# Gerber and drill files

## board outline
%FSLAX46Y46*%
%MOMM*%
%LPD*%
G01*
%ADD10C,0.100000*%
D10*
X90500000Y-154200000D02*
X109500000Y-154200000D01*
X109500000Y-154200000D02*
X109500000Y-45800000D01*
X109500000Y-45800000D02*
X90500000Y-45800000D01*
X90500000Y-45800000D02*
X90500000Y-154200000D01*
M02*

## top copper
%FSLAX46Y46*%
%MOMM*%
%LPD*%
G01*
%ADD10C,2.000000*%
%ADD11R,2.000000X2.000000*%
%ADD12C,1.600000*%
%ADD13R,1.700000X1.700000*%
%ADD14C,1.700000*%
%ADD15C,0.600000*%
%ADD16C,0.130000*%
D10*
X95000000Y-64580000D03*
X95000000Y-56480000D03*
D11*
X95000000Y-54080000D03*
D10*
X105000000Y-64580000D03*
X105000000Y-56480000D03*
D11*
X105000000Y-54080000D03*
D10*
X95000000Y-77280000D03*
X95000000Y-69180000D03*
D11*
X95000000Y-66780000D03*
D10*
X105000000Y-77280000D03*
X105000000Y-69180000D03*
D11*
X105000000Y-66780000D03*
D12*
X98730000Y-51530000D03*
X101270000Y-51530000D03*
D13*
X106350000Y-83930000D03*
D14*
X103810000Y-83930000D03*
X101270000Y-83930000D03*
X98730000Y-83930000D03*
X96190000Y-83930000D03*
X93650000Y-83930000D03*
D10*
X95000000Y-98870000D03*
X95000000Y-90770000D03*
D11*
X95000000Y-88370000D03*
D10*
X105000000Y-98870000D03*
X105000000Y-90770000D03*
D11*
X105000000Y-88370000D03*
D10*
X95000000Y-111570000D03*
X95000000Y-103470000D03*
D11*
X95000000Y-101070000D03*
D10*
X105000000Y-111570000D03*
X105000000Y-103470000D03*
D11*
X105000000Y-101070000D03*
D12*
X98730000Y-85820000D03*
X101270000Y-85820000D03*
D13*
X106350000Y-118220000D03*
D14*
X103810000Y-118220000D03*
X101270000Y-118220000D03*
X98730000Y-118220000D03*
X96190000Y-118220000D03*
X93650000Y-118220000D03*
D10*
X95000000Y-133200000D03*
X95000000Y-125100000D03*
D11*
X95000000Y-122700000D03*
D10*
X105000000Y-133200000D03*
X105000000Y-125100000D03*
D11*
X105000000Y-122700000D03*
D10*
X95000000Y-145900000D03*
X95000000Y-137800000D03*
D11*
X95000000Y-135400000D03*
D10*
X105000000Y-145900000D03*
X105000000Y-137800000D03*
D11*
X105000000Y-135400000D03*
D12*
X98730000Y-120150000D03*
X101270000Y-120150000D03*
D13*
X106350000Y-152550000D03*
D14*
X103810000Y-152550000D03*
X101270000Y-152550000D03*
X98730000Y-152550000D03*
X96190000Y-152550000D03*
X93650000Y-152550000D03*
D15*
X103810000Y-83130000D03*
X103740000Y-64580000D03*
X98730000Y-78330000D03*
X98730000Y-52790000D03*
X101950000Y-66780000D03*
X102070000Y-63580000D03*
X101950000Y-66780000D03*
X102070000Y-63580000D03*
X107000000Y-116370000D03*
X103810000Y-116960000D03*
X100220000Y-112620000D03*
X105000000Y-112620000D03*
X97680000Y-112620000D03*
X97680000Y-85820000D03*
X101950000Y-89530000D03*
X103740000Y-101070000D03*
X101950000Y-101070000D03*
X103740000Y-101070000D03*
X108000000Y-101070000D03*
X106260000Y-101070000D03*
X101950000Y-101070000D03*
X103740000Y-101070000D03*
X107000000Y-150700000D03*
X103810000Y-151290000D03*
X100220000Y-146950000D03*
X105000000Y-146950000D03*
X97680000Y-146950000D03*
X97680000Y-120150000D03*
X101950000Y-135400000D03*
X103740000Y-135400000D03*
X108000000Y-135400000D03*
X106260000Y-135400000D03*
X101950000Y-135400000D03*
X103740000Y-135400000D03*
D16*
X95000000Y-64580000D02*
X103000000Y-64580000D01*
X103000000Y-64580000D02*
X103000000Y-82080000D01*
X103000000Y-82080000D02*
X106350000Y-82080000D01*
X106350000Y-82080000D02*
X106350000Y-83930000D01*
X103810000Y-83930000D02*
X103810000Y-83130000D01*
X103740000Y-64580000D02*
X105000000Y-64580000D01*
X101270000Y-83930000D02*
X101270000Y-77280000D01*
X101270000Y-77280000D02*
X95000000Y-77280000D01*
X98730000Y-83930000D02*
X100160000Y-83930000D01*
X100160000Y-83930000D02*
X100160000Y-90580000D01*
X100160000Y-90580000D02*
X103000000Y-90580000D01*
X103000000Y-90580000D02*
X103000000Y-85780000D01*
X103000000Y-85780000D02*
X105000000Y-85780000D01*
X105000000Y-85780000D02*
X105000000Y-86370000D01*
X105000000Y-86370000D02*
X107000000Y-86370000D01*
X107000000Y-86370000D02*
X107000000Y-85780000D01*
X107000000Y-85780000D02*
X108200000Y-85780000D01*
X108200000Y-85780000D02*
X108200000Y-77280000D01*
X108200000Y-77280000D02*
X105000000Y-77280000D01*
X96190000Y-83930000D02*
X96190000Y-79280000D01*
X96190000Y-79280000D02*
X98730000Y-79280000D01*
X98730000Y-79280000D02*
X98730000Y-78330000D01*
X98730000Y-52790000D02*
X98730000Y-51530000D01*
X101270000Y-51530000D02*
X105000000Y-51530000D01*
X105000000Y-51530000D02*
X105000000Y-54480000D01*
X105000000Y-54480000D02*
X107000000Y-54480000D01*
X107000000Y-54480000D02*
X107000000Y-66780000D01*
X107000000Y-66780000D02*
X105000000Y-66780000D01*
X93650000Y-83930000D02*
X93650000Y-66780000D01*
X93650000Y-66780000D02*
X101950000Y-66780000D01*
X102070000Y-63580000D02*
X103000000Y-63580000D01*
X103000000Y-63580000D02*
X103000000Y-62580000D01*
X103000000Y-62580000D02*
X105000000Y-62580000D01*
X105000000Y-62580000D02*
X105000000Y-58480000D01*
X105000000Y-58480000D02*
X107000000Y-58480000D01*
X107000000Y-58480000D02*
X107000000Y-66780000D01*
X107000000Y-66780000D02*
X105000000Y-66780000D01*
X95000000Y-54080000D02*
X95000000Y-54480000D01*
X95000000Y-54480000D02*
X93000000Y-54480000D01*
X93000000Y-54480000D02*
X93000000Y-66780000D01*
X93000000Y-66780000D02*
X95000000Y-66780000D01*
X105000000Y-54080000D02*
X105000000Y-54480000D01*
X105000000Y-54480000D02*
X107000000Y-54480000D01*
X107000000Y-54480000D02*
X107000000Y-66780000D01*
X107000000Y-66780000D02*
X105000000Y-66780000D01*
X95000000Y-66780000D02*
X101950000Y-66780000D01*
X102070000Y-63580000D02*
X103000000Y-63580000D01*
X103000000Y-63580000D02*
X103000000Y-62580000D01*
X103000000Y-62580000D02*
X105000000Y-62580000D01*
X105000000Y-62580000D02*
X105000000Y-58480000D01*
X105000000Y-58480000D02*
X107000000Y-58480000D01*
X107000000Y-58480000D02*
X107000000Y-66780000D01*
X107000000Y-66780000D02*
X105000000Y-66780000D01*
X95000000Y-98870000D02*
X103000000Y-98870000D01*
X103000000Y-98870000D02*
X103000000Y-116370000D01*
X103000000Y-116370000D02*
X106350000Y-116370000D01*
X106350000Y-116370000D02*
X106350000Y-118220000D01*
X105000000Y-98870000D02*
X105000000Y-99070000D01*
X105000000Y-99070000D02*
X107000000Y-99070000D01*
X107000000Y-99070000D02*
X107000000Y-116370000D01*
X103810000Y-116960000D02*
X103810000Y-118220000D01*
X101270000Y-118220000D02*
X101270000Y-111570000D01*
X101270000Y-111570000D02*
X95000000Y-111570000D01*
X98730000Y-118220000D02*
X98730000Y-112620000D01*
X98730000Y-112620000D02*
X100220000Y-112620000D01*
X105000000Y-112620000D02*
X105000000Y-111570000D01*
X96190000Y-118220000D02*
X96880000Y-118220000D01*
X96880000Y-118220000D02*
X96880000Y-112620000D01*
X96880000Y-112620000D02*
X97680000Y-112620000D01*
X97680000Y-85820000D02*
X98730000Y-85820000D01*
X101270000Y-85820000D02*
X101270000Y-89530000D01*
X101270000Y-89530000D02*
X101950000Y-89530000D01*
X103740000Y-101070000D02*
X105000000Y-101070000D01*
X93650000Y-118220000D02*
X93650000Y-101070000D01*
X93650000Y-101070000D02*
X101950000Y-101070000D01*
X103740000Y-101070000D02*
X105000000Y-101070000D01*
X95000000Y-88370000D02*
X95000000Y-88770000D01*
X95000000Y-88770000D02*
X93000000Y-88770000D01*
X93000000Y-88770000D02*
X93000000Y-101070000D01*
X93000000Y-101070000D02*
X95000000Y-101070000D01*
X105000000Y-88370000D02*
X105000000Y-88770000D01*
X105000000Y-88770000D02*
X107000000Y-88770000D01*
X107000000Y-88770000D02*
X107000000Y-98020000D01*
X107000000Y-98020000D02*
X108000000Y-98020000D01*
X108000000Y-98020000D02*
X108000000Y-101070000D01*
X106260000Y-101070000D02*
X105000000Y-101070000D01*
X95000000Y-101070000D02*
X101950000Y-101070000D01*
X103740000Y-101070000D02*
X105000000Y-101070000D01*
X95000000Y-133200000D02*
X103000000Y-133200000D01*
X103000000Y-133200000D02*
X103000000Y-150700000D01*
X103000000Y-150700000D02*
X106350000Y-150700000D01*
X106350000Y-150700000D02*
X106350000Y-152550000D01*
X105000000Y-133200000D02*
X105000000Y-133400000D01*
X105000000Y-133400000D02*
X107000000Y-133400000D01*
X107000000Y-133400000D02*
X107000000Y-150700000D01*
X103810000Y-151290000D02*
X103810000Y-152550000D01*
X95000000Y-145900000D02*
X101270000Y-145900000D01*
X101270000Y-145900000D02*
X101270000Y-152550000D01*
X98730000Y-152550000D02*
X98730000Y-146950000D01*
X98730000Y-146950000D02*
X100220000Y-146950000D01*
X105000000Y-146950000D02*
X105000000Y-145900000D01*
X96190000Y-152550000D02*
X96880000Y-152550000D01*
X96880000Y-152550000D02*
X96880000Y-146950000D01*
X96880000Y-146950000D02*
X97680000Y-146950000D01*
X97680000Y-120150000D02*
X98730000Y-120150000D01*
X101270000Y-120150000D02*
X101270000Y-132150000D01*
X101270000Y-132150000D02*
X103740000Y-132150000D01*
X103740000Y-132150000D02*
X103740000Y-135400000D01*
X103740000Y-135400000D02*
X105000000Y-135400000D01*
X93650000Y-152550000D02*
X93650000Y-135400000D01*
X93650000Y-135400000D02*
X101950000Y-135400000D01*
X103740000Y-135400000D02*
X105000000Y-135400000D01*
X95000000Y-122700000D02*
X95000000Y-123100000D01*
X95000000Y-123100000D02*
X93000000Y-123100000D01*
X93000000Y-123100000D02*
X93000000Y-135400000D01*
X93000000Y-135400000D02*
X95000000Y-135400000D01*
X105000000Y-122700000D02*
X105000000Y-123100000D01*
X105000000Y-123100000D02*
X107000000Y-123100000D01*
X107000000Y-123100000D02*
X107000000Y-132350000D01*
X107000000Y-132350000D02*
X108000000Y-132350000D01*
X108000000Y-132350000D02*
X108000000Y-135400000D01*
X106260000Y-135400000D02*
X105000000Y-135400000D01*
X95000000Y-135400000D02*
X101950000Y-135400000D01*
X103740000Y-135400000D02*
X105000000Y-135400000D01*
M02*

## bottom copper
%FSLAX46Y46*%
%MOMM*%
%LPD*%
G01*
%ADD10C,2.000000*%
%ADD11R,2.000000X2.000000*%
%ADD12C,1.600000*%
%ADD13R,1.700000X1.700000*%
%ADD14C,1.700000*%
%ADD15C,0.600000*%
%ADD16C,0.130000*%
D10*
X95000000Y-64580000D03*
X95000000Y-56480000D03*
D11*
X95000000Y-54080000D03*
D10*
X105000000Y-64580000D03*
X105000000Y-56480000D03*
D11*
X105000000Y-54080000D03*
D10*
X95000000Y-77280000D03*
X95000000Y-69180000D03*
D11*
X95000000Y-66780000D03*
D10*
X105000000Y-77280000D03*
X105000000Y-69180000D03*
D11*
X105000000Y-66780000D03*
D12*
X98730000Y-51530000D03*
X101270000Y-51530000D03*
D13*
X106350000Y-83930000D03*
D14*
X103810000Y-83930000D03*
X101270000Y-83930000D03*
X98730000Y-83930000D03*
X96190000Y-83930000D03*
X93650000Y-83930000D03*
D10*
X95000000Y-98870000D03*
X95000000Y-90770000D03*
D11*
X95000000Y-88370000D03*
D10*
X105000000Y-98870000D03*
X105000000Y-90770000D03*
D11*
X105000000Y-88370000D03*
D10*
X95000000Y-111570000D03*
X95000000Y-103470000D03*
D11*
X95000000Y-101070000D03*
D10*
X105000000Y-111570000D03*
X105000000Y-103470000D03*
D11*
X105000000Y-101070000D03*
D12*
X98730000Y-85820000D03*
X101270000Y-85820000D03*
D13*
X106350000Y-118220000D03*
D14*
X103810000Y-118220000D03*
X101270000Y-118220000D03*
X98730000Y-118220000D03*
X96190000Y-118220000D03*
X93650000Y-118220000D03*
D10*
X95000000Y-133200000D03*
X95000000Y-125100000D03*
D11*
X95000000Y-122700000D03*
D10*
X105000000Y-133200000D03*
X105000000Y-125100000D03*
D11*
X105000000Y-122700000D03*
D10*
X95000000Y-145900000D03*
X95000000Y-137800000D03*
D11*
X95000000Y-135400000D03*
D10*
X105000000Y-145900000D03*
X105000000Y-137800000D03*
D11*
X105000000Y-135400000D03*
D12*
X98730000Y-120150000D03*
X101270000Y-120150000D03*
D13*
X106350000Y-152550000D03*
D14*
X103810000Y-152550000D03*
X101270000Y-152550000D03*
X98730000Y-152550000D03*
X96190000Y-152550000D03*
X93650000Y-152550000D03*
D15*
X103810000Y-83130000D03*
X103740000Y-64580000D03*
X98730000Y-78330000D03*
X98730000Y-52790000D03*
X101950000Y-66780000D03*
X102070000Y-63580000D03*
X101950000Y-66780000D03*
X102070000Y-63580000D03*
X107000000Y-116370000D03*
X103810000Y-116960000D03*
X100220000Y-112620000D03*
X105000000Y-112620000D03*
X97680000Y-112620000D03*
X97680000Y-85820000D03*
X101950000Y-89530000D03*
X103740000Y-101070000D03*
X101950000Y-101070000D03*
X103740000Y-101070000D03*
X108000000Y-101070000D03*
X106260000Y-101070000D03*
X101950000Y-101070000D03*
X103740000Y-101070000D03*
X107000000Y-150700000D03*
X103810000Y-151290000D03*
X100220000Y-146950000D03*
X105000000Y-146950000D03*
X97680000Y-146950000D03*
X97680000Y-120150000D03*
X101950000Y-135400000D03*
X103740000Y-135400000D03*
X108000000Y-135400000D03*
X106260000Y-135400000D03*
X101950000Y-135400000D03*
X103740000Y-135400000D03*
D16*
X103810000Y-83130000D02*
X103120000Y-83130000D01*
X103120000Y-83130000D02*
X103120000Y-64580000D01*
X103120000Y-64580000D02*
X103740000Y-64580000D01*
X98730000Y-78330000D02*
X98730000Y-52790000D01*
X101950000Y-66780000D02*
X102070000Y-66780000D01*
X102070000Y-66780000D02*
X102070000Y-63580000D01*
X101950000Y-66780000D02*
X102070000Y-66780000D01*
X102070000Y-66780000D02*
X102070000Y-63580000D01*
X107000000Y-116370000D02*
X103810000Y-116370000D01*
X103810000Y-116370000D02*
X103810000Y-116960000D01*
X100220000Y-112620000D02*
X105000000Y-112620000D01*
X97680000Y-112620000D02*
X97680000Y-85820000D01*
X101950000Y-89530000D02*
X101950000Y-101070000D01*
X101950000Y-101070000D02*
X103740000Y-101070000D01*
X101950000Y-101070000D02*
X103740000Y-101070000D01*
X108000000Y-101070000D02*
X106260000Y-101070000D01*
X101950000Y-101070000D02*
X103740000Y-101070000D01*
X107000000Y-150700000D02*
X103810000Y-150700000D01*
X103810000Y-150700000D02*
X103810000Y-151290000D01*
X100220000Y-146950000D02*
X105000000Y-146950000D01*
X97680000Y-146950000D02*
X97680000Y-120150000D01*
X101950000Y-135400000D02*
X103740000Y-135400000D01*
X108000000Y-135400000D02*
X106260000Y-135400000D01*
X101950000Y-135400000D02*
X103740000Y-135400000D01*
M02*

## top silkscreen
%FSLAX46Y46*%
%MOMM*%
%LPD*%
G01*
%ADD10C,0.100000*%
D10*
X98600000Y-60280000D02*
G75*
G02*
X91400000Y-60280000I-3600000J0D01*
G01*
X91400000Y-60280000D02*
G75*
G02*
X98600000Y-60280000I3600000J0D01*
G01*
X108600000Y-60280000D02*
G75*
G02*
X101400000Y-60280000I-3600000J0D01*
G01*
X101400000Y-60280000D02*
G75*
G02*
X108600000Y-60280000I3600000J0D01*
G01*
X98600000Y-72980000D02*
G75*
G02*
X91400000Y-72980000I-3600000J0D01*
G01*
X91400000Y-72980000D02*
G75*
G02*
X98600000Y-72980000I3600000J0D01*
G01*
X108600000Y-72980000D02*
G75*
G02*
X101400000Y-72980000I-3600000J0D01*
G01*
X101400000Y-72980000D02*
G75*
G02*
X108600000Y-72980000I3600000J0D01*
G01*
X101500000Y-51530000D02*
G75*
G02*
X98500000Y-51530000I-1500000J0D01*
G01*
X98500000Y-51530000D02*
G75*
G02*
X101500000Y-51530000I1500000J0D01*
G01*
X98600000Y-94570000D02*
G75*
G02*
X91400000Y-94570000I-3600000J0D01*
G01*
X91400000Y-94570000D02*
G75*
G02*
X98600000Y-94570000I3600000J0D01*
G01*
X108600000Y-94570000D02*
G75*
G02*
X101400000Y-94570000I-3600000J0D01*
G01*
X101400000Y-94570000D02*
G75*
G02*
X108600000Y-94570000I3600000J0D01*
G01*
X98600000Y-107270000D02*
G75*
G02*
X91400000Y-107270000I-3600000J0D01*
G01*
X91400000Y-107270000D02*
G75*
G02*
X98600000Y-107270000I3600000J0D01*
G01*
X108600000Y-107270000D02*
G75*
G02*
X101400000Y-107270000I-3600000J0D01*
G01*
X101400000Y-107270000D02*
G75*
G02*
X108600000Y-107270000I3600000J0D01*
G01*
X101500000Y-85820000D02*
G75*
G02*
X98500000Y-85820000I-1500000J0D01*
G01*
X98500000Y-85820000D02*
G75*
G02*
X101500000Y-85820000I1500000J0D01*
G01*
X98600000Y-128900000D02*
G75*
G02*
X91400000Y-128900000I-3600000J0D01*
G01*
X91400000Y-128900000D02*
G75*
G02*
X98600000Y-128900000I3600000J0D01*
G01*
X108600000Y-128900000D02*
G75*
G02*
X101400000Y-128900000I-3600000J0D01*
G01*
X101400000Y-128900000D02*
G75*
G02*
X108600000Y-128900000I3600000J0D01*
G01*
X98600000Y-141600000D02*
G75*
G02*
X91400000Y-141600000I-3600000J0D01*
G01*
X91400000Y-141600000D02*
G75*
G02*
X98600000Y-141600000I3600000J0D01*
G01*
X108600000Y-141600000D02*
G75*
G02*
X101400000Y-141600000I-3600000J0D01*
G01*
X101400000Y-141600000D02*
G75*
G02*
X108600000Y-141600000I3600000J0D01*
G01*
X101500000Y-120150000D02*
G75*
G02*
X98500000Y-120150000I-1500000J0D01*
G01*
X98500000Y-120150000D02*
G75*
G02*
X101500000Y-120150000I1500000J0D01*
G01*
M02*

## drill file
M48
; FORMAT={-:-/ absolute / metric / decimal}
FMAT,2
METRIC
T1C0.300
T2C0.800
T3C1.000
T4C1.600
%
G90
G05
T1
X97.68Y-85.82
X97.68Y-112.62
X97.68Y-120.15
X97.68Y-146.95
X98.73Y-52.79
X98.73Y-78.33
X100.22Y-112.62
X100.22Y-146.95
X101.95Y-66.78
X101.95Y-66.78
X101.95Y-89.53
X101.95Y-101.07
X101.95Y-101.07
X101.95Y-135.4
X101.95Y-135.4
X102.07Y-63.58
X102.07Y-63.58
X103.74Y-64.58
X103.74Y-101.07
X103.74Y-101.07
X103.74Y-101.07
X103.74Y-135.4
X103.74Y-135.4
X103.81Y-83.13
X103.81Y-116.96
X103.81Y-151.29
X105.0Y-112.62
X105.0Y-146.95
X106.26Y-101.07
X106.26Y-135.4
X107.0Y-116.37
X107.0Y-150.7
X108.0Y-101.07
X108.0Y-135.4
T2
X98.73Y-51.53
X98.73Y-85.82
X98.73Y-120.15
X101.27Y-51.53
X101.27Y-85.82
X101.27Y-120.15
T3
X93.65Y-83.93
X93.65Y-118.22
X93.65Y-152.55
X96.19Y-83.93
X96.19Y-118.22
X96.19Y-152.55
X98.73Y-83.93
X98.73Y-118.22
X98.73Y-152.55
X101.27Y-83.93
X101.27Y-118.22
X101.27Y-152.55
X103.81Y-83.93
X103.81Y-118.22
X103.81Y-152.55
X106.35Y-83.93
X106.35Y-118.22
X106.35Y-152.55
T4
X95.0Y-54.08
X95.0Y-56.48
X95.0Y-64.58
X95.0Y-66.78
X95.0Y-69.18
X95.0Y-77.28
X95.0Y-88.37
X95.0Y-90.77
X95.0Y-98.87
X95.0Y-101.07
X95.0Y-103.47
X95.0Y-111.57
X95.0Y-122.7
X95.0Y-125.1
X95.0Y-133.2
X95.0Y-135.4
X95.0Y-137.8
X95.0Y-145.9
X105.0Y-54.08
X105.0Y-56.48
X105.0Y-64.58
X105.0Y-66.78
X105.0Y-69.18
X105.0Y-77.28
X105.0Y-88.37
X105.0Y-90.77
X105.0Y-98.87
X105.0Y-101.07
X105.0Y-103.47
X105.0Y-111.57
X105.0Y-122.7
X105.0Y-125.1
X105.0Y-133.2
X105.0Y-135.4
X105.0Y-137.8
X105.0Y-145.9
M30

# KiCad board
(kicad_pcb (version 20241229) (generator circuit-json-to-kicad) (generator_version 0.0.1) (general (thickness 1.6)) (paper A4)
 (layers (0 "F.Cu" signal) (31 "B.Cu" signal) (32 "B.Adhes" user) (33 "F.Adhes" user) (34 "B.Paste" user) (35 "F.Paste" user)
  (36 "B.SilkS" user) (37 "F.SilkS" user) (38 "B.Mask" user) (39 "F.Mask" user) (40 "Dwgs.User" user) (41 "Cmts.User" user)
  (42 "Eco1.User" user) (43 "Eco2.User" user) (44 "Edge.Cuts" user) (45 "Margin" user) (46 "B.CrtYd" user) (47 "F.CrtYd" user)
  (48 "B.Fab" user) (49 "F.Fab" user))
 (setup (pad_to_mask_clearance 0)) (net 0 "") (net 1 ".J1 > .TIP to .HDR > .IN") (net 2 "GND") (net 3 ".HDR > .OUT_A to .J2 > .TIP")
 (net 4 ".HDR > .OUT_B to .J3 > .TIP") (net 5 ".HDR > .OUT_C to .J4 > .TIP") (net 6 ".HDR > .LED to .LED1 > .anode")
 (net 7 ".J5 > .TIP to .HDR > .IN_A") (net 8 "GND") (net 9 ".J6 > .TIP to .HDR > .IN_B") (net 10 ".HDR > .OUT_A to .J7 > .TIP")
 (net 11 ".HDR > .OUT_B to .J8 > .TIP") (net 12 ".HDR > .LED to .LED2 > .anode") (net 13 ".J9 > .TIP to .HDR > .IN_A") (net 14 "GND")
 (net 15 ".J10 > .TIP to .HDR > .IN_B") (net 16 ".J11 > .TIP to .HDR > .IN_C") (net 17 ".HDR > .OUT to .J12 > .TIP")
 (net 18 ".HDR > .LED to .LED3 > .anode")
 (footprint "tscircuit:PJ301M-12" (layer F.Cu) (at 95 59.33 0)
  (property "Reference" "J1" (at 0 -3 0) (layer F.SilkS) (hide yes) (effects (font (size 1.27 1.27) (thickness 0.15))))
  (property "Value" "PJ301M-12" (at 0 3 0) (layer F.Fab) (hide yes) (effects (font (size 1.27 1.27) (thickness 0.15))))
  (fp_circle (center 0 0.9500000000000028) (end 3.6 0.9500000000000028) (layer F.SilkS) (stroke (width 0.1) (type default)) (fill no))
  (pad "1" thru_hole circle (at 0 5.25 0) (size 2 2) (drill 1.6) (layers *.Cu *.Mask) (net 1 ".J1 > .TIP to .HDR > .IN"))
  (pad "2" thru_hole circle (at 0 -2.8499999999999943 0) (size 2 2) (drill 1.6) (layers *.Cu *.Mask))
  (pad "3" thru_hole rect (at 0 -5.25 0) (size 2 2) (drill 1.6) (layers *.Cu *.Mask) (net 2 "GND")))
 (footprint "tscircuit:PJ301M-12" (layer F.Cu) (at 105 59.33 0)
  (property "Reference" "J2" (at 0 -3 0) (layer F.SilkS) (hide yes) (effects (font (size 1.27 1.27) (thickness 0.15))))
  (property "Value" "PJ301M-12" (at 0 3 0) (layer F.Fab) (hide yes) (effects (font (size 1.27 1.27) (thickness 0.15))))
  (fp_circle (center 0 0.9500000000000028) (end 3.6 0.9500000000000028) (layer F.SilkS) (stroke (width 0.1) (type default)) (fill no))
  (pad "1" thru_hole circle (at 0 5.25 0) (size 2 2) (drill 1.6) (layers *.Cu *.Mask) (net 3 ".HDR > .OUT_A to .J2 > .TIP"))
  (pad "2" thru_hole circle (at 0 -2.8499999999999943 0) (size 2 2) (drill 1.6) (layers *.Cu *.Mask))
  (pad "3" thru_hole rect (at 0 -5.25 0) (size 2 2) (drill 1.6) (layers *.Cu *.Mask) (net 2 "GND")))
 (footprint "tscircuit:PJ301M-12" (layer F.Cu) (at 95 72.03 0)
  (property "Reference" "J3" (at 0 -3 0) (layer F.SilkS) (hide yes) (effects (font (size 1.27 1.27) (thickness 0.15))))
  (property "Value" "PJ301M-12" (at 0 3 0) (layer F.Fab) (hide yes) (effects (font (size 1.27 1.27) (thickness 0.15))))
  (fp_circle (center 0 0.9500000000000028) (end 3.6 0.9500000000000028) (layer F.SilkS) (stroke (width 0.1) (type default)) (fill no))
  (pad "1" thru_hole circle (at 0 5.2500000000000036 0) (size 2 2) (drill 1.6) (layers *.Cu *.Mask) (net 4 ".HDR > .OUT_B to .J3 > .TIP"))
  (pad "2" thru_hole circle (at 0 -2.849999999999998 0) (size 2 2) (drill 1.6) (layers *.Cu *.Mask))
  (pad "3" thru_hole rect (at 0 -5.25 0) (size 2 2) (drill 1.6) (layers *.Cu *.Mask) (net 2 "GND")))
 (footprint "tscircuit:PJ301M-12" (layer F.Cu) (at 105 72.03 0)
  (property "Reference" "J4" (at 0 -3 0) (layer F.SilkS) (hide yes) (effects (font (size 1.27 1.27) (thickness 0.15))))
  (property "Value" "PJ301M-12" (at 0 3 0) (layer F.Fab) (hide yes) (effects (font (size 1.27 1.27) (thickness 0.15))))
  (fp_circle (center 0 0.9500000000000028) (end 3.6 0.9500000000000028) (layer F.SilkS) (stroke (width 0.1) (type default)) (fill no))
  (pad "1" thru_hole circle (at 0 5.2500000000000036 0) (size 2 2) (drill 1.6) (layers *.Cu *.Mask) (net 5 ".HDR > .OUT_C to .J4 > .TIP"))
  (pad "2" thru_hole circle (at 0 -2.849999999999998 0) (size 2 2) (drill 1.6) (layers *.Cu *.Mask))
  (pad "3" thru_hole rect (at 0 -5.25 0) (size 2 2) (drill 1.6) (layers *.Cu *.Mask) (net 2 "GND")))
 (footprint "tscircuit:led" (layer F.Cu) (at 100 51.53 0)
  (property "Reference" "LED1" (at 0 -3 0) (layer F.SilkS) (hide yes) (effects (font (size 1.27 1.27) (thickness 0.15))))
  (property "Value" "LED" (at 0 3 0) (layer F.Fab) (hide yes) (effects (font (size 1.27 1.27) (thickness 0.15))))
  (fp_circle (center 0 0) (end 1.5 0) (layer F.SilkS) (stroke (width 0.1) (type default)) (fill no))
  (pad "1" thru_hole circle (at -1.27 0 0) (size 1.6 1.6) (drill 0.8) (layers *.Cu *.Mask) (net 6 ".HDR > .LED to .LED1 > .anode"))
  (pad "2" thru_hole circle (at 1.27 0 0) (size 1.6 1.6) (drill 0.8) (layers *.Cu *.Mask) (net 2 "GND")))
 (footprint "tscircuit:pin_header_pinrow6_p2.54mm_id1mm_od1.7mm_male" (layer F.Cu) (at 100 83.93 0)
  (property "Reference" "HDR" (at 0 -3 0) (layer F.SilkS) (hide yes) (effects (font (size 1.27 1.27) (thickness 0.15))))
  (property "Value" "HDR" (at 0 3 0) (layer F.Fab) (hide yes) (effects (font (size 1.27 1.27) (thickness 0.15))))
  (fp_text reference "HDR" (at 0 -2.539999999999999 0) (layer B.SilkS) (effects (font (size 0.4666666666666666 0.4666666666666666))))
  (pad "1" thru_hole rect (at 6.35 0 180) (size 1.7 1.7) (drill 1) (layers *.Cu *.Mask) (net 1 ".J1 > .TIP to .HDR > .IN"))
  (pad "2" thru_hole circle (at 3.8099999999999996 0 0) (size 1.7 1.7) (drill 1) (layers *.Cu *.Mask) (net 3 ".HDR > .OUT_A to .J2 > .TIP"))
  (pad "3" thru_hole circle (at 1.2699999999999996 0 0) (size 1.7 1.7) (drill 1) (layers *.Cu *.Mask) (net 4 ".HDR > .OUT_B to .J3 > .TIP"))
  (pad "4" thru_hole circle (at -1.2700000000000005 0 0) (size 1.7 1.7) (drill 1) (layers *.Cu *.Mask) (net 5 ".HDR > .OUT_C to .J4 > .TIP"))
  (pad "5" thru_hole circle (at -3.8100000000000005 0 0) (size 1.7 1.7) (drill 1) (layers *.Cu *.Mask)
   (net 6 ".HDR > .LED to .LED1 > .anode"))
  (pad "6" thru_hole circle (at -6.35 0 0) (size 1.7 1.7) (drill 1) (layers *.Cu *.Mask) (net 2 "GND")))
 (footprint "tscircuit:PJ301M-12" (layer F.Cu) (at 95 93.62 0)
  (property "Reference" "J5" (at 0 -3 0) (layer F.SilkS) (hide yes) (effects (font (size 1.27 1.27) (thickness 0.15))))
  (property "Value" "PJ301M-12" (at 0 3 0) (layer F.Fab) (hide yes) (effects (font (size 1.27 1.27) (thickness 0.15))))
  (fp_circle (center 0 0.9499999999999993) (end 3.6 0.9499999999999993) (layer F.SilkS) (stroke (width 0.1) (type default)) (fill no))
  (pad "1" thru_hole circle (at 0 5.249999999999999 0) (size 2 2) (drill 1.6) (layers *.Cu *.Mask) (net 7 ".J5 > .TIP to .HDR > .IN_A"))
  (pad "2" thru_hole circle (at 0 -2.8500000000000014 0) (size 2 2) (drill 1.6) (layers *.Cu *.Mask))
  (pad "3" thru_hole rect (at 0 -5.25 0) (size 2 2) (drill 1.6) (layers *.Cu *.Mask) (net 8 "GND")))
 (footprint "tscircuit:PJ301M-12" (layer F.Cu) (at 105 93.62 0)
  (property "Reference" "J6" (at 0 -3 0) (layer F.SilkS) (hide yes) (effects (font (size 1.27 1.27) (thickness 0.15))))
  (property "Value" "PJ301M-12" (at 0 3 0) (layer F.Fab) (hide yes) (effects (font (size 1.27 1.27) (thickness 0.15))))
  (fp_circle (center 0 0.9499999999999993) (end 3.6 0.9499999999999993) (layer F.SilkS) (stroke (width 0.1) (type default)) (fill no))
  (pad "1" thru_hole circle (at 0 5.249999999999999 0) (size 2 2) (drill 1.6) (layers *.Cu *.Mask) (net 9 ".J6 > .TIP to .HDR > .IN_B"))
  (pad "2" thru_hole circle (at 0 -2.8500000000000014 0) (size 2 2) (drill 1.6) (layers *.Cu *.Mask))
  (pad "3" thru_hole rect (at 0 -5.25 0) (size 2 2) (drill 1.6) (layers *.Cu *.Mask) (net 8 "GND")))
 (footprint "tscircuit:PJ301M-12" (layer F.Cu) (at 95 106.32 0)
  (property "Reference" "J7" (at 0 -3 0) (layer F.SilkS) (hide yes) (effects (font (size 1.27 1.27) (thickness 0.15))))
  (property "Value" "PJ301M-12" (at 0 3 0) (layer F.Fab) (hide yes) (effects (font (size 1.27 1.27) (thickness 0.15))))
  (fp_circle (center 0 0.9499999999999993) (end 3.6 0.9499999999999993) (layer F.SilkS) (stroke (width 0.1) (type default)) (fill no))
  (pad "1" thru_hole circle (at 0 5.25 0) (size 2 2) (drill 1.6) (layers *.Cu *.Mask) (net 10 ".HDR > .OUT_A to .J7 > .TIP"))
  (pad "2" thru_hole circle (at 0 -2.8500000000000005 0) (size 2 2) (drill 1.6) (layers *.Cu *.Mask))
  (pad "3" thru_hole rect (at 0 -5.250000000000001 0) (size 2 2) (drill 1.6) (layers *.Cu *.Mask) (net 8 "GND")))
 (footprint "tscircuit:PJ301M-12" (layer F.Cu) (at 105 106.32 0)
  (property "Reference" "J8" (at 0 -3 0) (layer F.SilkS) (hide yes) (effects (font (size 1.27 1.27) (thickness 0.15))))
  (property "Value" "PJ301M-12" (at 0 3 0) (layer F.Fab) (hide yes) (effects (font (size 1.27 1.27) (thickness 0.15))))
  (fp_circle (center 0 0.9499999999999993) (end 3.6 0.9499999999999993) (layer F.SilkS) (stroke (width 0.1) (type default)) (fill no))
  (pad "1" thru_hole circle (at 0 5.25 0) (size 2 2) (drill 1.6) (layers *.Cu *.Mask) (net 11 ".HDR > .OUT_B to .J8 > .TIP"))
  (pad "2" thru_hole circle (at 0 -2.8500000000000005 0) (size 2 2) (drill 1.6) (layers *.Cu *.Mask))
  (pad "3" thru_hole rect (at 0 -5.250000000000001 0) (size 2 2) (drill 1.6) (layers *.Cu *.Mask) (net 8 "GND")))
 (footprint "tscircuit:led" (layer F.Cu) (at 100 85.82 0)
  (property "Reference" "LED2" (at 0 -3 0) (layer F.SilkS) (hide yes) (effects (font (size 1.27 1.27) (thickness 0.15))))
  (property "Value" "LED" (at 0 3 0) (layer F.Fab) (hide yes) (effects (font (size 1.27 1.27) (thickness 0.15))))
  (fp_circle (center 0 0) (end 1.5 0) (layer F.SilkS) (stroke (width 0.1) (type default)) (fill no))
  (pad "1" thru_hole circle (at -1.27 0 0) (size 1.6 1.6) (drill 0.8) (layers *.Cu *.Mask) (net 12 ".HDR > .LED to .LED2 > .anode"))
  (pad "2" thru_hole circle (at 1.27 0 0) (size 1.6 1.6) (drill 0.8) (layers *.Cu *.Mask) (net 8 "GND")))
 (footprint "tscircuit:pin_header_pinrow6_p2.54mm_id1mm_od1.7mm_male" (layer F.Cu) (at 100 118.22 0)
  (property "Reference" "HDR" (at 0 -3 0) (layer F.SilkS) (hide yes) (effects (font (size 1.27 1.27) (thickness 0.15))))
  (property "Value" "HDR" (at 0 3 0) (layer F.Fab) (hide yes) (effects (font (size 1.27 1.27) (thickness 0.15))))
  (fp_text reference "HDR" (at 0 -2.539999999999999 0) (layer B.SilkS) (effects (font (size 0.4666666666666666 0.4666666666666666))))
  (pad "1" thru_hole rect (at 6.35 0 180) (size 1.7 1.7) (drill 1) (layers *.Cu *.Mask) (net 7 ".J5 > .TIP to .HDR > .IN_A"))
  (pad "2" thru_hole circle (at 3.8099999999999996 0 0) (size 1.7 1.7) (drill 1) (layers *.Cu *.Mask) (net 9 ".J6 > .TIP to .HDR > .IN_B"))
  (pad "3" thru_hole circle (at 1.2699999999999996 0 0) (size 1.7 1.7) (drill 1) (layers *.Cu *.Mask) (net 10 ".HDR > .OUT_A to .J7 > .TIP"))
  (pad "4" thru_hole circle (at -1.2700000000000005 0 0) (size 1.7 1.7) (drill 1) (layers *.Cu *.Mask)
   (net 11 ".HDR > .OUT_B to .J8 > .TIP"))
  (pad "5" thru_hole circle (at -3.8100000000000005 0 0) (size 1.7 1.7) (drill 1) (layers *.Cu *.Mask)
   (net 12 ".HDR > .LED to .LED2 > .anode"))
  (pad "6" thru_hole circle (at -6.35 0 0) (size 1.7 1.7) (drill 1) (layers *.Cu *.Mask) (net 8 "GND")))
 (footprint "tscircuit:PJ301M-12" (layer F.Cu) (at 95 127.94999999999999 0)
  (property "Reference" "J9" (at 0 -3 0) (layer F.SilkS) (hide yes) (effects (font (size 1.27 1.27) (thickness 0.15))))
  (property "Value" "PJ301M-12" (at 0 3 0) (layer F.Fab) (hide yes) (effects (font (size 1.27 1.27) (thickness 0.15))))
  (fp_circle (center 0 0.9500000000000028) (end 3.6 0.9500000000000028) (layer F.SilkS) (stroke (width 0.1) (type default)) (fill no))
  (pad "1" thru_hole circle (at 0 5.25 0) (size 2 2) (drill 1.6) (layers *.Cu *.Mask) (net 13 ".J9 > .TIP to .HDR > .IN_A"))
  (pad "2" thru_hole circle (at 0 -2.849999999999998 0) (size 2 2) (drill 1.6) (layers *.Cu *.Mask))
  (pad "3" thru_hole rect (at 0 -5.2499999999999964 0) (size 2 2) (drill 1.6) (layers *.Cu *.Mask) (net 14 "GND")))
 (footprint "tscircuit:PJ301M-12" (layer F.Cu) (at 105 127.94999999999999 0)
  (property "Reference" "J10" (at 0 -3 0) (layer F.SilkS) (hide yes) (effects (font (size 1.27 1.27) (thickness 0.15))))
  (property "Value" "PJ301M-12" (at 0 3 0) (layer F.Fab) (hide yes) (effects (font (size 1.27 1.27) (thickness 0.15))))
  (fp_circle (center 0 0.9500000000000028) (end 3.6 0.9500000000000028) (layer F.SilkS) (stroke (width 0.1) (type default)) (fill no))
  (pad "1" thru_hole circle (at 0 5.25 0) (size 2 2) (drill 1.6) (layers *.Cu *.Mask) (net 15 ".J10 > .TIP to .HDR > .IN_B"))
  (pad "2" thru_hole circle (at 0 -2.849999999999998 0) (size 2 2) (drill 1.6) (layers *.Cu *.Mask))
  (pad "3" thru_hole rect (at 0 -5.2499999999999964 0) (size 2 2) (drill 1.6) (layers *.Cu *.Mask) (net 14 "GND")))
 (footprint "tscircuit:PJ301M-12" (layer F.Cu) (at 95 140.65 0)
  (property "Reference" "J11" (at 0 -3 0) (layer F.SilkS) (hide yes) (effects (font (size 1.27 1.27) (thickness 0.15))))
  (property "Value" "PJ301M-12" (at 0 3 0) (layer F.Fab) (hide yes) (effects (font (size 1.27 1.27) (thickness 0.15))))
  (fp_circle (center 0 0.9500000000000028) (end 3.6 0.9500000000000028) (layer F.SilkS) (stroke (width 0.1) (type default)) (fill no))
  (pad "1" thru_hole circle (at 0 5.25 0) (size 2 2) (drill 1.6) (layers *.Cu *.Mask) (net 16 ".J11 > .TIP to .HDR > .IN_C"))
  (pad "2" thru_hole circle (at 0 -2.8499999999999943 0) (size 2 2) (drill 1.6) (layers *.Cu *.Mask))
  (pad "3" thru_hole rect (at 0 -5.25 0) (size 2 2) (drill 1.6) (layers *.Cu *.Mask) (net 14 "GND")))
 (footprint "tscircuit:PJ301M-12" (layer F.Cu) (at 105 140.65 0)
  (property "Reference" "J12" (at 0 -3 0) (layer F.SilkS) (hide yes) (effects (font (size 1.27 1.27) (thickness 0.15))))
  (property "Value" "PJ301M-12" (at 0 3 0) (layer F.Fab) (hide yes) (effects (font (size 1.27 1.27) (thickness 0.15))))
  (fp_circle (center 0 0.9500000000000028) (end 3.6 0.9500000000000028) (layer F.SilkS) (stroke (width 0.1) (type default)) (fill no))
  (pad "1" thru_hole circle (at 0 5.25 0) (size 2 2) (drill 1.6) (layers *.Cu *.Mask) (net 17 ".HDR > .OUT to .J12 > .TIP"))
  (pad "2" thru_hole circle (at 0 -2.8499999999999943 0) (size 2 2) (drill 1.6) (layers *.Cu *.Mask))
  (pad "3" thru_hole rect (at 0 -5.25 0) (size 2 2) (drill 1.6) (layers *.Cu *.Mask) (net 14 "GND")))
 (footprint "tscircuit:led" (layer F.Cu) (at 100 120.15 0)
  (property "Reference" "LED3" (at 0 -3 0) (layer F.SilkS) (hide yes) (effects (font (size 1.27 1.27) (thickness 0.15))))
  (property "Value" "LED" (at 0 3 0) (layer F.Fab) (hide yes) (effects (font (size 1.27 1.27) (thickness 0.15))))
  (fp_circle (center 0 0) (end 1.5 0) (layer F.SilkS) (stroke (width 0.1) (type default)) (fill no))
  (pad "1" thru_hole circle (at -1.27 0 0) (size 1.6 1.6) (drill 0.8) (layers *.Cu *.Mask) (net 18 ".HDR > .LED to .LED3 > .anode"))
  (pad "2" thru_hole circle (at 1.27 0 0) (size 1.6 1.6) (drill 0.8) (layers *.Cu *.Mask) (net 14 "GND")))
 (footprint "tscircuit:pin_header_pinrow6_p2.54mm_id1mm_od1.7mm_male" (layer F.Cu) (at 100 152.55 0)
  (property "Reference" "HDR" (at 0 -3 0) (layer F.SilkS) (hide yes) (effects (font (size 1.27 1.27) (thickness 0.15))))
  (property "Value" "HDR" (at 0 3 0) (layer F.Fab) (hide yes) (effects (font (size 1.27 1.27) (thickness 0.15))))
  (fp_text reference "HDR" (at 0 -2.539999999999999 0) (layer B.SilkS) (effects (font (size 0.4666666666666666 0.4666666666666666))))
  (pad "1" thru_hole rect (at 6.35 0 180) (size 1.7 1.7) (drill 1) (layers *.Cu *.Mask) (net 13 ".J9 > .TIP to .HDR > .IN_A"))
  (pad "2" thru_hole circle (at 3.8099999999999996 0 0) (size 1.7 1.7) (drill 1) (layers *.Cu *.Mask) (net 15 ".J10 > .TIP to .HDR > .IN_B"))
  (pad "3" thru_hole circle (at 1.2699999999999996 0 0) (size 1.7 1.7) (drill 1) (layers *.Cu *.Mask) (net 16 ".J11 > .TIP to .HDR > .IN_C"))
  (pad "4" thru_hole circle (at -1.2700000000000005 0 0) (size 1.7 1.7) (drill 1) (layers *.Cu *.Mask) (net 17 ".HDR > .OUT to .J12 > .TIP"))
  (pad "5" thru_hole circle (at -3.8100000000000005 0 0) (size 1.7 1.7) (drill 1) (layers *.Cu *.Mask)
   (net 18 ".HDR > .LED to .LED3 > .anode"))
  (pad "6" thru_hole circle (at -6.35 0 0) (size 1.7 1.7) (drill 1) (layers *.Cu *.Mask) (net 14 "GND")))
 (segment (start 95 64.58) (end 103 64.58) (width 0.13) (layer F.Cu) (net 1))
 (segment (start 103 64.58) (end 103 82.08) (width 0.13) (layer F.Cu) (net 1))
 (segment (start 103 82.08) (end 106.35 82.08) (width 0.13) (layer F.Cu) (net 1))
 (segment (start 106.35 82.08) (end 106.35 83.93) (width 0.13) (layer F.Cu) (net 1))
 (segment (start 103.81 83.93) (end 103.81 83.13) (width 0.13) (layer F.Cu) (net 3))
 (segment (start 103.81 83.13) (end 103.12 83.13) (width 0.13) (layer B.Cu) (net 3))
 (segment (start 103.12 83.13) (end 103.12 64.58) (width 0.13) (layer B.Cu) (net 3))
 (segment (start 103.12 64.58) (end 103.74 64.58) (width 0.13) (layer B.Cu) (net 3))
 (segment (start 103.74 64.58) (end 105 64.58) (width 0.13) (layer F.Cu) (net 3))
 (segment (start 101.27 83.93) (end 101.27 77.28) (width 0.13) (layer F.Cu) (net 4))
 (segment (start 101.27 77.28) (end 95 77.28) (width 0.13) (layer F.Cu) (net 4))
 (segment (start 98.73 83.93) (end 100.16 83.93) (width 0.13) (layer F.Cu) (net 5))
 (segment (start 100.16 83.93) (end 100.16 90.58) (width 0.13) (layer F.Cu) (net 5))
 (segment (start 100.16 90.58) (end 103 90.58) (width 0.13) (layer F.Cu) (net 5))
 (segment (start 103 90.58) (end 103 85.78) (width 0.13) (layer F.Cu) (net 5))
 (segment (start 103 85.78) (end 105 85.78) (width 0.13) (layer F.Cu) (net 5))
 (segment (start 105 85.78) (end 105 86.37) (width 0.13) (layer F.Cu) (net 5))
 (segment (start 105 86.37) (end 107 86.37) (width 0.13) (layer F.Cu) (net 5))
 (segment (start 107 86.37) (end 107 85.78) (width 0.13) (layer F.Cu) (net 5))
 (segment (start 107 85.78) (end 108.2 85.78) (width 0.13) (layer F.Cu) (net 5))
 (segment (start 108.2 85.78) (end 108.2 77.28) (width 0.13) (layer F.Cu) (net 5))
 (segment (start 108.2 77.28) (end 105 77.28) (width 0.13) (layer F.Cu) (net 5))
 (segment (start 96.19 83.93) (end 96.19 79.28) (width 0.13) (layer F.Cu) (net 6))
 (segment (start 96.19 79.28) (end 98.73 79.28) (width 0.13) (layer F.Cu) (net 6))
 (segment (start 98.73 79.28) (end 98.73 78.33000000000001) (width 0.13) (layer F.Cu) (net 6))
 (segment (start 98.73 78.33000000000001) (end 98.73 52.790000000000006) (width 0.13) (layer B.Cu) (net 6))
 (segment (start 98.73 52.790000000000006) (end 98.73 51.53) (width 0.13) (layer F.Cu) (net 6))
 (segment (start 101.27 51.53) (end 105 51.53) (width 0.13) (layer F.Cu) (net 2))
 (segment (start 105 51.53) (end 105 54.480000000000004) (width 0.13) (layer F.Cu) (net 2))
 (segment (start 105 54.480000000000004) (end 107 54.480000000000004) (width 0.13) (layer F.Cu) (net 2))
 (segment (start 107 54.480000000000004) (end 107 66.78) (width 0.13) (layer F.Cu) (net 2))
 (segment (start 107 66.78) (end 105 66.78) (width 0.13) (layer F.Cu) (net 2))
 (segment (start 93.65 83.93) (end 93.65 66.78) (width 0.13) (layer F.Cu) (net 2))
 (segment (start 93.65 66.78) (end 101.95 66.78) (width 0.13) (layer F.Cu) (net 2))
 (segment (start 101.95 66.78) (end 102.07 66.78) (width 0.13) (layer B.Cu) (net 2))
 (segment (start 102.07 66.78) (end 102.07 63.58) (width 0.13) (layer B.Cu) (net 2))
 (segment (start 102.07 63.58) (end 103 63.58) (width 0.13) (layer F.Cu) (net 2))
 (segment (start 103 63.58) (end 103 62.58) (width 0.13) (layer F.Cu) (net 2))
 (segment (start 103 62.58) (end 105 62.58) (width 0.13) (layer F.Cu) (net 2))
 (segment (start 105 62.58) (end 105 58.480000000000004) (width 0.13) (layer F.Cu) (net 2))
 (segment (start 105 58.480000000000004) (end 107 58.480000000000004) (width 0.13) (layer F.Cu) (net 2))
 (segment (start 107 58.480000000000004) (end 107 66.78) (width 0.13) (layer F.Cu) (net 2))
 (segment (start 107 66.78) (end 105 66.78) (width 0.13) (layer F.Cu) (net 2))
 (segment (start 95 54.08) (end 95 54.480000000000004) (width 0.13) (layer F.Cu) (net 2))
 (segment (start 95 54.480000000000004) (end 93 54.480000000000004) (width 0.13) (layer F.Cu) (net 2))
 (segment (start 93 54.480000000000004) (end 93 66.78) (width 0.13) (layer F.Cu) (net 2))
 (segment (start 93 66.78) (end 95 66.78) (width 0.13) (layer F.Cu) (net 2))
 (segment (start 105 54.08) (end 105 54.480000000000004) (width 0.13) (layer F.Cu) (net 2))
 (segment (start 105 54.480000000000004) (end 107 54.480000000000004) (width 0.13) (layer F.Cu) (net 2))
 (segment (start 107 54.480000000000004) (end 107 66.78) (width 0.13) (layer F.Cu) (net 2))
 (segment (start 107 66.78) (end 105 66.78) (width 0.13) (layer F.Cu) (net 2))
 (segment (start 95 66.78) (end 101.95 66.78) (width 0.13) (layer F.Cu) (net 2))
 (segment (start 101.95 66.78) (end 102.07 66.78) (width 0.13) (layer B.Cu) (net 2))
 (segment (start 102.07 66.78) (end 102.07 63.58) (width 0.13) (layer B.Cu) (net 2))
 (segment (start 102.07 63.58) (end 103 63.58) (width 0.13) (layer F.Cu) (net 2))
 (segment (start 103 63.58) (end 103 62.58) (width 0.13) (layer F.Cu) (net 2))
 (segment (start 103 62.58) (end 105 62.58) (width 0.13) (layer F.Cu) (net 2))
 (segment (start 105 62.58) (end 105 58.480000000000004) (width 0.13) (layer F.Cu) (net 2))
 (segment (start 105 58.480000000000004) (end 107 58.480000000000004) (width 0.13) (layer F.Cu) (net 2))
 (segment (start 107 58.480000000000004) (end 107 66.78) (width 0.13) (layer F.Cu) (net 2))
 (segment (start 107 66.78) (end 105 66.78) (width 0.13) (layer F.Cu) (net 2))
 (segment (start 95 98.87) (end 103 98.87) (width 0.13) (layer F.Cu) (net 7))
 (segment (start 103 98.87) (end 103 116.37) (width 0.13) (layer F.Cu) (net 7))
 (segment (start 103 116.37) (end 106.35 116.37) (width 0.13) (layer F.Cu) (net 7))
 (segment (start 106.35 116.37) (end 106.35 118.22) (width 0.13) (layer F.Cu) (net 7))
 (segment (start 105 98.87) (end 105 99.07) (width 0.13) (layer F.Cu) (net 9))
 (segment (start 105 99.07) (end 107 99.07) (width 0.13) (layer F.Cu) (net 9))
 (segment (start 107 99.07) (end 107 116.37) (width 0.13) (layer F.Cu) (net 9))
 (segment (start 107 116.37) (end 103.81 116.37) (width 0.13) (layer B.Cu) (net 9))
 (segment (start 103.81 116.37) (end 103.81 116.96000000000001) (width 0.13) (layer B.Cu) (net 9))
 (segment (start 103.81 116.96000000000001) (end 103.81 118.22) (width 0.13) (layer F.Cu) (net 9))
 (segment (start 101.27 118.22) (end 101.27 111.57) (width 0.13) (layer F.Cu) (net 10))
 (segment (start 101.27 111.57) (end 95 111.57) (width 0.13) (layer F.Cu) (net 10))
 (segment (start 98.73 118.22) (end 98.73 112.62) (width 0.13) (layer F.Cu) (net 11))
 (segment (start 98.73 112.62) (end 100.22 112.62) (width 0.13) (layer F.Cu) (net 11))
 (segment (start 100.22 112.62) (end 105 112.62) (width 0.13) (layer B.Cu) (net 11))
 (segment (start 105 112.62) (end 105 111.57) (width 0.13) (layer F.Cu) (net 11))
 (segment (start 96.19 118.22) (end 96.88 118.22) (width 0.13) (layer F.Cu) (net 12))
 (segment (start 96.88 118.22) (end 96.88 112.62) (width 0.13) (layer F.Cu) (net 12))
 (segment (start 96.88 112.62) (end 97.68 112.62) (width 0.13) (layer F.Cu) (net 12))
 (segment (start 97.68 112.62) (end 97.68 85.82) (width 0.13) (layer B.Cu) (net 12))
 (segment (start 97.68 85.82) (end 98.73 85.82) (width 0.13) (layer F.Cu) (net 12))
 (segment (start 101.27 85.82) (end 101.27 89.53) (width 0.13) (layer F.Cu) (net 8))
 (segment (start 101.27 89.53) (end 101.95 89.53) (width 0.13) (layer F.Cu) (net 8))
 (segment (start 101.95 89.53) (end 101.95 101.07) (width 0.13) (layer B.Cu) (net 8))
 (segment (start 101.95 101.07) (end 103.74 101.07) (width 0.13) (layer B.Cu) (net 8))
 (segment (start 103.74 101.07) (end 105 101.07) (width 0.13) (layer F.Cu) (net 8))
 (segment (start 93.65 118.22) (end 93.65 101.07) (width 0.13) (layer F.Cu) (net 8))
 (segment (start 93.65 101.07) (end 101.95 101.07) (width 0.13) (layer F.Cu) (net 8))
 (segment (start 101.95 101.07) (end 103.74 101.07) (width 0.13) (layer B.Cu) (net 8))
 (segment (start 103.74 101.07) (end 105 101.07) (width 0.13) (layer F.Cu) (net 8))
 (segment (start 95 88.37) (end 95 88.77) (width 0.13) (layer F.Cu) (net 8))
 (segment (start 95 88.77) (end 93 88.77) (width 0.13) (layer F.Cu) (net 8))
 (segment (start 93 88.77) (end 93 101.07) (width 0.13) (layer F.Cu) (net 8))
 (segment (start 93 101.07) (end 95 101.07) (width 0.13) (layer F.Cu) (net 8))
 (segment (start 105 88.37) (end 105 88.77) (width 0.13) (layer F.Cu) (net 8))
 (segment (start 105 88.77) (end 107 88.77) (width 0.13) (layer F.Cu) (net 8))
 (segment (start 107 88.77) (end 107 98.02) (width 0.13) (layer F.Cu) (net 8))
 (segment (start 107 98.02) (end 108 98.02) (width 0.13) (layer F.Cu) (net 8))
 (segment (start 108 98.02) (end 108 101.07) (width 0.13) (layer F.Cu) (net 8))
 (segment (start 108 101.07) (end 106.26 101.07) (width 0.13) (layer B.Cu) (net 8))
 (segment (start 106.26 101.07) (end 105 101.07) (width 0.13) (layer F.Cu) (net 8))
 (segment (start 95 101.07) (end 101.95 101.07) (width 0.13) (layer F.Cu) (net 8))
 (segment (start 101.95 101.07) (end 103.74 101.07) (width 0.13) (layer B.Cu) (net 8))
 (segment (start 103.74 101.07) (end 105 101.07) (width 0.13) (layer F.Cu) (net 8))
 (segment (start 95 133.2) (end 103 133.2) (width 0.13) (layer F.Cu) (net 13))
 (segment (start 103 133.2) (end 103 150.7) (width 0.13) (layer F.Cu) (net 13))
 (segment (start 103 150.7) (end 106.35 150.7) (width 0.13) (layer F.Cu) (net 13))
 (segment (start 106.35 150.7) (end 106.35 152.55) (width 0.13) (layer F.Cu) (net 13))
 (segment (start 105 133.2) (end 105 133.4) (width 0.13) (layer F.Cu) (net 15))
 (segment (start 105 133.4) (end 107 133.4) (width 0.13) (layer F.Cu) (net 15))
 (segment (start 107 133.4) (end 107 150.7) (width 0.13) (layer F.Cu) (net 15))
 (segment (start 107 150.7) (end 103.81 150.7) (width 0.13) (layer B.Cu) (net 15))
 (segment (start 103.81 150.7) (end 103.81 151.29) (width 0.13) (layer B.Cu) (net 15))
 (segment (start 103.81 151.29) (end 103.81 152.55) (width 0.13) (layer F.Cu) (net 15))
 (segment (start 95 145.9) (end 101.27 145.9) (width 0.13) (layer F.Cu) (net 16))
 (segment (start 101.27 145.9) (end 101.27 152.55) (width 0.13) (layer F.Cu) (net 16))
 (segment (start 98.73 152.55) (end 98.73 146.95) (width 0.13) (layer F.Cu) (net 17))
 (segment (start 98.73 146.95) (end 100.22 146.95) (width 0.13) (layer F.Cu) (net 17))
 (segment (start 100.22 146.95) (end 105 146.95) (width 0.13) (layer B.Cu) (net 17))
 (segment (start 105 146.95) (end 105 145.9) (width 0.13) (layer F.Cu) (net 17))
 (segment (start 96.19 152.55) (end 96.88 152.55) (width 0.13) (layer F.Cu) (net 18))
 (segment (start 96.88 152.55) (end 96.88 146.95) (width 0.13) (layer F.Cu) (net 18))
 (segment (start 96.88 146.95) (end 97.68 146.95) (width 0.13) (layer F.Cu) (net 18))
 (segment (start 97.68 146.95) (end 97.68 120.15) (width 0.13) (layer B.Cu) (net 18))
 (segment (start 97.68 120.15) (end 98.73 120.15) (width 0.13) (layer F.Cu) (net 18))
 (segment (start 101.27 120.15) (end 101.27 132.15) (width 0.13) (layer F.Cu) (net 14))
 (segment (start 101.27 132.15) (end 103.74 132.15) (width 0.13) (layer F.Cu) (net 14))
 (segment (start 103.74 132.15) (end 103.74 135.4) (width 0.13) (layer F.Cu) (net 14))
 (segment (start 103.74 135.4) (end 105 135.4) (width 0.13) (layer F.Cu) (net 14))
 (segment (start 93.65 152.55) (end 93.65 135.4) (width 0.13) (layer F.Cu) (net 14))
 (segment (start 93.65 135.4) (end 101.95 135.4) (width 0.13) (layer F.Cu) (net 14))
 (segment (start 101.95 135.4) (end 103.74 135.4) (width 0.13) (layer B.Cu) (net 14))
 (segment (start 103.74 135.4) (end 105 135.4) (width 0.13) (layer F.Cu) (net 14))
 (segment (start 95 122.7) (end 95 123.1) (width 0.13) (layer F.Cu) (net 14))
 (segment (start 95 123.1) (end 93 123.1) (width 0.13) (layer F.Cu) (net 14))
 (segment (start 93 123.1) (end 93 135.4) (width 0.13) (layer F.Cu) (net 14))
 (segment (start 93 135.4) (end 95 135.4) (width 0.13) (layer F.Cu) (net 14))
 (segment (start 105 122.7) (end 105 123.1) (width 0.13) (layer F.Cu) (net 14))
 (segment (start 105 123.1) (end 107 123.1) (width 0.13) (layer F.Cu) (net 14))
 (segment (start 107 123.1) (end 107 132.35) (width 0.13) (layer F.Cu) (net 14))
 (segment (start 107 132.35) (end 108 132.35) (width 0.13) (layer F.Cu) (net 14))
 (segment (start 108 132.35) (end 108 135.4) (width 0.13) (layer F.Cu) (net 14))
 (segment (start 108 135.4) (end 106.26 135.4) (width 0.13) (layer B.Cu) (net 14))
 (segment (start 106.26 135.4) (end 105 135.4) (width 0.13) (layer F.Cu) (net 14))
 (segment (start 95 135.4) (end 101.95 135.4) (width 0.13) (layer F.Cu) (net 14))
 (segment (start 101.95 135.4) (end 103.74 135.4) (width 0.13) (layer B.Cu) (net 14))
 (segment (start 103.74 135.4) (end 105 135.4) (width 0.13) (layer F.Cu) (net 14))
 (gr_line (start 90.5 154.2) (end 109.5 154.2) (width 0.1) (layer Edge.Cuts))
 (gr_line (start 109.5 154.2) (end 109.5 45.8) (width 0.1) (layer Edge.Cuts))
 (gr_line (start 109.5 45.8) (end 90.5 45.8) (width 0.1) (layer Edge.Cuts))
 (gr_line (start 90.5 45.8) (end 90.5 154.2) (width 0.1) (layer Edge.Cuts))
 (via (at 103.81 83.13) (size 0.6) (drill 0.3) (layers F.Cu B.Cu) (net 3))
 (via (at 103.74 64.58) (size 0.6) (drill 0.3) (layers F.Cu B.Cu) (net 3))
 (via (at 98.73 78.33000000000001) (size 0.6) (drill 0.3) (layers F.Cu B.Cu) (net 6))
 (via (at 98.73 52.790000000000006) (size 0.6) (drill 0.3) (layers F.Cu B.Cu) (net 6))
 (via (at 101.95 66.78) (size 0.6) (drill 0.3) (layers F.Cu B.Cu) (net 2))
 (via (at 102.07 63.58) (size 0.6) (drill 0.3) (layers F.Cu B.Cu) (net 2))
 (via (at 101.95 66.78) (size 0.6) (drill 0.3) (layers F.Cu B.Cu) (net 2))
 (via (at 102.07 63.58) (size 0.6) (drill 0.3) (layers F.Cu B.Cu) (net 2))
 (via (at 107 116.37) (size 0.6) (drill 0.3) (layers F.Cu B.Cu) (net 9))
 (via (at 103.81 116.96000000000001) (size 0.6) (drill 0.3) (layers F.Cu B.Cu) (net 9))
 (via (at 100.22 112.62) (size 0.6) (drill 0.3) (layers F.Cu B.Cu) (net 11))
 (via (at 105 112.62) (size 0.6) (drill 0.3) (layers F.Cu B.Cu) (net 11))
 (via (at 97.68 112.62) (size 0.6) (drill 0.3) (layers F.Cu B.Cu) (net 12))
 (via (at 97.68 85.82) (size 0.6) (drill 0.3) (layers F.Cu B.Cu) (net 12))
 (via (at 101.95 89.53) (size 0.6) (drill 0.3) (layers F.Cu B.Cu) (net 8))
 (via (at 103.74 101.07) (size 0.6) (drill 0.3) (layers F.Cu B.Cu) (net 8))
 (via (at 101.95 101.07) (size 0.6) (drill 0.3) (layers F.Cu B.Cu) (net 8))
 (via (at 103.74 101.07) (size 0.6) (drill 0.3) (layers F.Cu B.Cu) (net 8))
 (via (at 108 101.07) (size 0.6) (drill 0.3) (layers F.Cu B.Cu) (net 8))
 (via (at 106.26 101.07) (size 0.6) (drill 0.3) (layers F.Cu B.Cu) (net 8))
 (via (at 101.95 101.07) (size 0.6) (drill 0.3) (layers F.Cu B.Cu) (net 8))
 (via (at 103.74 101.07) (size 0.6) (drill 0.3) (layers F.Cu B.Cu) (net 8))
 (via (at 107 150.7) (size 0.6) (drill 0.3) (layers F.Cu B.Cu) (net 15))
 (via (at 103.81 151.29) (size 0.6) (drill 0.3) (layers F.Cu B.Cu) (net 15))
 (via (at 100.22 146.95) (size 0.6) (drill 0.3) (layers F.Cu B.Cu) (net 17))
 (via (at 105 146.95) (size 0.6) (drill 0.3) (layers F.Cu B.Cu) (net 17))
 (via (at 97.68 146.95) (size 0.6) (drill 0.3) (layers F.Cu B.Cu) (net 18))
 (via (at 97.68 120.15) (size 0.6) (drill 0.3) (layers F.Cu B.Cu) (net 18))
 (via (at 101.95 135.4) (size 0.6) (drill 0.3) (layers F.Cu B.Cu) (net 14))
 (via (at 103.74 135.4) (size 0.6) (drill 0.3) (layers F.Cu B.Cu) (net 14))
 (via (at 108 135.4) (size 0.6) (drill 0.3) (layers F.Cu B.Cu) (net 14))
 (via (at 106.26 135.4) (size 0.6) (drill 0.3) (layers F.Cu B.Cu) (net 14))
 (via (at 101.95 135.4) (size 0.6) (drill 0.3) (layers F.Cu B.Cu) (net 14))
 (via (at 103.74 135.4) (size 0.6) (drill 0.3) (layers F.Cu B.Cu) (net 14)))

